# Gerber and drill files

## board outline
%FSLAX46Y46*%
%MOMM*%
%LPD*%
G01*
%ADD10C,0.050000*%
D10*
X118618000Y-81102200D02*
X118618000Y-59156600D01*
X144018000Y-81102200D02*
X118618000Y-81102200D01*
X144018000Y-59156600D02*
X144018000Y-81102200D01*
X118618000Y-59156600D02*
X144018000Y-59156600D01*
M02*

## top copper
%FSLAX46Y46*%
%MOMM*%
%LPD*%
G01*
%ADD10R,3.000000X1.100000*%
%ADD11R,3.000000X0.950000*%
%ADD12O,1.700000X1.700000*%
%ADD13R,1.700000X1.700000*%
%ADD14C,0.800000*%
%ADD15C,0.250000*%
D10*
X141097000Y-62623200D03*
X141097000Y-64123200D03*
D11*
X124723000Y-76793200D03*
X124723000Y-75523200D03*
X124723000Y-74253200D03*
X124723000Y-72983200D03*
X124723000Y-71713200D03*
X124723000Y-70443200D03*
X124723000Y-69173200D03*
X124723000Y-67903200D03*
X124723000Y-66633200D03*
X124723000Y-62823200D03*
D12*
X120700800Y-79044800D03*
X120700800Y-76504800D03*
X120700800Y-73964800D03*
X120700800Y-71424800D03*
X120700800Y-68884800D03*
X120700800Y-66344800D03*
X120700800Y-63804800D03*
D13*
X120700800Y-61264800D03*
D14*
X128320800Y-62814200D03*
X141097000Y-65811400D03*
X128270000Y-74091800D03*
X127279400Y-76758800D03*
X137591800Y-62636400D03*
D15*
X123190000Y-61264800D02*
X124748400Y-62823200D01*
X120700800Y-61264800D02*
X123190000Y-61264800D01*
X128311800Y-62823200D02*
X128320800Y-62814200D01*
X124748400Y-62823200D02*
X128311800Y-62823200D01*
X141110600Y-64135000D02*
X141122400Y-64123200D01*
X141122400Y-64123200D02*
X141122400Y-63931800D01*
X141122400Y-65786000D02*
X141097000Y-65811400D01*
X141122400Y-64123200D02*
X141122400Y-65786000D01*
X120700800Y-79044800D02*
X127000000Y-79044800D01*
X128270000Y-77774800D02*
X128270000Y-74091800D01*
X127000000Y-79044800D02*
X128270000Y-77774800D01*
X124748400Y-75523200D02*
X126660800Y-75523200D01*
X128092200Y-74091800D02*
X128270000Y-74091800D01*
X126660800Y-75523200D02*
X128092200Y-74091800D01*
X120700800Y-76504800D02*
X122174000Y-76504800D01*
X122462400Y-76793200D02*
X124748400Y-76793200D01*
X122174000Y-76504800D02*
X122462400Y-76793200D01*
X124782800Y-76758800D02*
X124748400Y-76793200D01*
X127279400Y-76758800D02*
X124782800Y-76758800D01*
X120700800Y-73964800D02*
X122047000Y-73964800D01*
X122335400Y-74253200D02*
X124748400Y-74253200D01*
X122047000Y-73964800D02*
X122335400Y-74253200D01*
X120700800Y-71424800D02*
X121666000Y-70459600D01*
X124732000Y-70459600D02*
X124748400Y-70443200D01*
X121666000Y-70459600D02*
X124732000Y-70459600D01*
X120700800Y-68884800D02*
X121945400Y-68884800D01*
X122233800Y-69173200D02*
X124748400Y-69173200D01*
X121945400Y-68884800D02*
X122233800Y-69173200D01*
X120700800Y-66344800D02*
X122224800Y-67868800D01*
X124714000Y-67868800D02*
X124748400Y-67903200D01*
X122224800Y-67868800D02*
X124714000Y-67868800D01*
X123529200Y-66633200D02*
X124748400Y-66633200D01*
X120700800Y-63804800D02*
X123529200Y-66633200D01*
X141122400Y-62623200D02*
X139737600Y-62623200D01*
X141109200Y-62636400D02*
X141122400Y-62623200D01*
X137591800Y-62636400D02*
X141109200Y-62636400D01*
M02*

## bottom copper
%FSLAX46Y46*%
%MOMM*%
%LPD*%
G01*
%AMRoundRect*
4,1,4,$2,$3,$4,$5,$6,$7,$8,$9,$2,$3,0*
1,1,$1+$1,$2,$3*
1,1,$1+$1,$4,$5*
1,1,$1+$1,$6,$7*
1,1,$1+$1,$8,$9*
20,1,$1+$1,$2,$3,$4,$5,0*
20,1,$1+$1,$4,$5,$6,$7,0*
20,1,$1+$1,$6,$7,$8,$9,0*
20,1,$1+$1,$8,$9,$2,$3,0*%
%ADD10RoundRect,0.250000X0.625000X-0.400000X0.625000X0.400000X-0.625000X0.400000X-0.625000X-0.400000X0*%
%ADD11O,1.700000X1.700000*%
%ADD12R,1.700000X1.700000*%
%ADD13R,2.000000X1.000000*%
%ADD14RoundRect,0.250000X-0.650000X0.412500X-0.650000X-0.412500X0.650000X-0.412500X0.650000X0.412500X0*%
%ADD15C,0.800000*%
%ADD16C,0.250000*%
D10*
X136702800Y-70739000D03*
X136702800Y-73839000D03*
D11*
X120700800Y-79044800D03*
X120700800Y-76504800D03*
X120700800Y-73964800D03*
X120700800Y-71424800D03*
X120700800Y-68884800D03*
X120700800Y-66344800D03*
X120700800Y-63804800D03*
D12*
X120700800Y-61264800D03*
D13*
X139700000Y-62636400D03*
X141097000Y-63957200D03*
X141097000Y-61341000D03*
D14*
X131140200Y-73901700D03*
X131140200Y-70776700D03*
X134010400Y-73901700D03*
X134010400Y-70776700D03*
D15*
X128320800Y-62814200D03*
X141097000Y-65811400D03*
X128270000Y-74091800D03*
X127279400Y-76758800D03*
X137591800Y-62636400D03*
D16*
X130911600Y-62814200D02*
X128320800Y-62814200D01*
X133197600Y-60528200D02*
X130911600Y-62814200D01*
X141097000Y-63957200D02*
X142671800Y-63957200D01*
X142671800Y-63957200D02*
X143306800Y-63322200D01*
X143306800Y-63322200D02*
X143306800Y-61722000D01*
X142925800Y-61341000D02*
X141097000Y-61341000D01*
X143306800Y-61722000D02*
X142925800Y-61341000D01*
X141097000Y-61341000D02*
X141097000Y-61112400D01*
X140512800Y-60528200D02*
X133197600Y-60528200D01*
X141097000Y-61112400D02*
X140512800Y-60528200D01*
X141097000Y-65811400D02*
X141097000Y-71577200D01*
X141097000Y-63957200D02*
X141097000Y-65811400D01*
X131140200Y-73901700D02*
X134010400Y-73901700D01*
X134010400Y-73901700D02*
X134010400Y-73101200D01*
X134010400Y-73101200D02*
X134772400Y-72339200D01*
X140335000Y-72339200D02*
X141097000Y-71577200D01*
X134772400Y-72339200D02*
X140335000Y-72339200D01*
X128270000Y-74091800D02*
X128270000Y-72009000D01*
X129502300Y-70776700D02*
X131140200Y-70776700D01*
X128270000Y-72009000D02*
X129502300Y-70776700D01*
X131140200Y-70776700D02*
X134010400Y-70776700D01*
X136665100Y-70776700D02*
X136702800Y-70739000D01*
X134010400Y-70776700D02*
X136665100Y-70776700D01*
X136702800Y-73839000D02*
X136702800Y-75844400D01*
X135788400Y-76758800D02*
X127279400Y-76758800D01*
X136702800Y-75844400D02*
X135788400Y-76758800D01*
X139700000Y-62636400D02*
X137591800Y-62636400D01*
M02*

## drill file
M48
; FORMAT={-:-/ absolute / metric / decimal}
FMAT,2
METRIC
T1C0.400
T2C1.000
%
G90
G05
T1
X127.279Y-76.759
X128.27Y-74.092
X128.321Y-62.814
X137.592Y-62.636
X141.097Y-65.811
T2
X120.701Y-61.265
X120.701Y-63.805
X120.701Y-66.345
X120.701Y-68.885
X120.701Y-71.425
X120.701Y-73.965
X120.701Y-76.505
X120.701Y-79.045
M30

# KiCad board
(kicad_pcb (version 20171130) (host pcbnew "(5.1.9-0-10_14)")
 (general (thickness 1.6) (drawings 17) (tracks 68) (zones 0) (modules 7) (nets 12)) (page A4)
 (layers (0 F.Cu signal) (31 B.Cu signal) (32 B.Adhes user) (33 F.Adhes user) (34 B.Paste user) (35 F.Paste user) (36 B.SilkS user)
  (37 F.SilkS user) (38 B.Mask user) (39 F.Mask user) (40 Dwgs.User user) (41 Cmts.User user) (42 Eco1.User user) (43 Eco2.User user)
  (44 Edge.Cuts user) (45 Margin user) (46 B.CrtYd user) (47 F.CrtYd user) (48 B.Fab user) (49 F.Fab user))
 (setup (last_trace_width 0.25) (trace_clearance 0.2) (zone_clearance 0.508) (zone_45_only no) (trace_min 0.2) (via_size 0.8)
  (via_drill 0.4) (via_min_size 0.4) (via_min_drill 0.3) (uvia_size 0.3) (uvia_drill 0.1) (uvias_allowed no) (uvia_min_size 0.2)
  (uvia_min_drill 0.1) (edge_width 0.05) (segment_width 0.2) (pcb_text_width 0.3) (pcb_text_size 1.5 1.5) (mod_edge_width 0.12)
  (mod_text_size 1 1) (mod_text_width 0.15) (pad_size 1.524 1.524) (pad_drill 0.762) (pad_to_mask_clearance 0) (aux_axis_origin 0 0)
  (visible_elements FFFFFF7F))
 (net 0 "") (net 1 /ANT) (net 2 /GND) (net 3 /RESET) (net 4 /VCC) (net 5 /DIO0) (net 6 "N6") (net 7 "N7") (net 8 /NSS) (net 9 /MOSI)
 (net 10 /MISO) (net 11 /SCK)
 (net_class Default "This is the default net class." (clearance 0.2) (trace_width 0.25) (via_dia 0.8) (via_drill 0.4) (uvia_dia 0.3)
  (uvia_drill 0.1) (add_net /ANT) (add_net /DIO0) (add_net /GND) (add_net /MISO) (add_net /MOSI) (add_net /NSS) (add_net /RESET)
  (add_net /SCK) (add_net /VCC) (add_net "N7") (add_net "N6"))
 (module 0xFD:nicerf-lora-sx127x (layer F.Cu) (at 133.223 71.3232)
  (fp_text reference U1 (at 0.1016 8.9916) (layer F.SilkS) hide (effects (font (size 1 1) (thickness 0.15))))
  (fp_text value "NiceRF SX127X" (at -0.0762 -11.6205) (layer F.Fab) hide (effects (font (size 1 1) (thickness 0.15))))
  (pad 13 smd rect (at 7.874 -8.7) (size 3 1.1) (layers F.Cu F.Paste F.Mask) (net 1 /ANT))
  (pad 14 smd rect (at 7.874 -7.2) (size 3 1.1) (layers F.Cu F.Paste F.Mask) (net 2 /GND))
  (pad 12 smd rect (at -8.5 5.47) (size 3 0.95) (layers F.Cu F.Paste F.Mask) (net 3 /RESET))
  (pad 11 smd rect (at -8.5 4.2) (size 3 0.95) (layers F.Cu F.Paste F.Mask) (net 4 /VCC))
  (pad 10 smd rect (at -8.5 2.93) (size 3 0.95) (layers F.Cu F.Paste F.Mask) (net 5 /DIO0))
  (pad 9 smd rect (at -8.5 1.66) (size 3 0.95) (layers F.Cu F.Paste F.Mask) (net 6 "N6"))
  (pad 8 smd rect (at -8.5 0.39) (size 3 0.95) (layers F.Cu F.Paste F.Mask) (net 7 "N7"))
  (pad 7 smd rect (at -8.5 -0.88) (size 3 0.95) (layers F.Cu F.Paste F.Mask) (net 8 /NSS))
  (pad 6 smd rect (at -8.5 -2.15) (size 3 0.95) (layers F.Cu F.Paste F.Mask) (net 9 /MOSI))
  (pad 5 smd rect (at -8.5 -3.42) (size 3 0.95) (layers F.Cu F.Paste F.Mask) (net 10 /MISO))
  (pad 4 smd rect (at -8.5 -4.69) (size 3 0.95) (layers F.Cu F.Paste F.Mask) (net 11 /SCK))
  (pad 1 smd rect (at -8.5 -8.5) (size 3 0.95) (layers F.Cu F.Paste F.Mask) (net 2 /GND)))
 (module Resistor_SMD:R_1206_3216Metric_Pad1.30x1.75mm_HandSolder (layer B.Cu) (at 136.7028 72.289 90)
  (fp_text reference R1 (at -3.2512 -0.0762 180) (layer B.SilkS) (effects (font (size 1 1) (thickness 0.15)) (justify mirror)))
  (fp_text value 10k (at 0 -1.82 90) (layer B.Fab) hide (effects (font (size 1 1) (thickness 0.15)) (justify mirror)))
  (pad 2 smd roundrect (at 1.55 0 90) (size 1.3 1.75) (layers B.Cu B.Paste B.Mask) (roundrect_rratio 0.192308) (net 4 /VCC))
  (pad 1 smd roundrect (at -1.55 0 90) (size 1.3 1.75) (layers B.Cu B.Paste B.Mask) (roundrect_rratio 0.192308) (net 3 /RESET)))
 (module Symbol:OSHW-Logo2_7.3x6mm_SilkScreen (layer B.Cu) (at 132.9944 64.2366 180)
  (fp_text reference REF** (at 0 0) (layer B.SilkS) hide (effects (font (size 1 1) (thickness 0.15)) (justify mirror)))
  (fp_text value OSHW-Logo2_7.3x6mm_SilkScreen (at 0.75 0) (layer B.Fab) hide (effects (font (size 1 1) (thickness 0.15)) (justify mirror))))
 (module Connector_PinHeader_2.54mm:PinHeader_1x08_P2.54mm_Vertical (layer F.Cu) (at 120.7008 61.2648)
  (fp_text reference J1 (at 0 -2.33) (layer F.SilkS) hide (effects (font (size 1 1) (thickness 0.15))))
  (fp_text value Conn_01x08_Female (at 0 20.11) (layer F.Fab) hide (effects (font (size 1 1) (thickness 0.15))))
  (pad 8 thru_hole oval (at 0 17.78) (size 1.7 1.7) (drill 1) (layers *.Cu *.Mask) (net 4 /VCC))
  (pad 7 thru_hole oval (at 0 15.24) (size 1.7 1.7) (drill 1) (layers *.Cu *.Mask) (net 3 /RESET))
  (pad 6 thru_hole oval (at 0 12.7) (size 1.7 1.7) (drill 1) (layers *.Cu *.Mask) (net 5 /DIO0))
  (pad 5 thru_hole oval (at 0 10.16) (size 1.7 1.7) (drill 1) (layers *.Cu *.Mask) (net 8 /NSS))
  (pad 4 thru_hole oval (at 0 7.62) (size 1.7 1.7) (drill 1) (layers *.Cu *.Mask) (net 9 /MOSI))
  (pad 3 thru_hole oval (at 0 5.08) (size 1.7 1.7) (drill 1) (layers *.Cu *.Mask) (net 10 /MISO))
  (pad 2 thru_hole oval (at 0 2.54) (size 1.7 1.7) (drill 1) (layers *.Cu *.Mask) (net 11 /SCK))
  (pad 1 thru_hole rect (at 0 0) (size 1.7 1.7) (drill 1) (layers *.Cu *.Mask) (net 2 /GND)))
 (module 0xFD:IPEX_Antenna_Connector (layer B.Cu) (at 141.097 62.6618 270)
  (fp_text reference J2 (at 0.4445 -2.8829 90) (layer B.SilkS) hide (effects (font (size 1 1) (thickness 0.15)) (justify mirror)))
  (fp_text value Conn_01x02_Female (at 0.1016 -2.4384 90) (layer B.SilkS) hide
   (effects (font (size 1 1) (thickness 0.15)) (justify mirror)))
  (pad 2 smd rect (at -0.0254 1.397) (size 2 1) (layers B.Cu B.Paste B.Mask) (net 1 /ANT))
  (pad 1 smd rect (at 1.2954 0 270) (size 1 2) (layers B.Cu B.Paste B.Mask) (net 2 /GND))
  (pad 1 smd rect (at -1.3208 0) (size 2 1) (layers B.Cu B.Paste B.Mask) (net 2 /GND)))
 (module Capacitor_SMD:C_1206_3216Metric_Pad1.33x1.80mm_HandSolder (layer B.Cu) (at 131.1402 72.3392 270)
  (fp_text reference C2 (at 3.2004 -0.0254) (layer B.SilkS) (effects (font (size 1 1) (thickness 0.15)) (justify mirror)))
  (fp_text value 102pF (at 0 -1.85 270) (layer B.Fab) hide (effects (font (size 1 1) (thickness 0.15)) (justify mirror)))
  (pad 2 smd roundrect (at 1.5625 0 270) (size 1.325 1.8) (layers B.Cu B.Paste B.Mask) (roundrect_rratio 0.188679) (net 2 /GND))
  (pad 1 smd roundrect (at -1.5625 0 270) (size 1.325 1.8) (layers B.Cu B.Paste B.Mask) (roundrect_rratio 0.188679) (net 4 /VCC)))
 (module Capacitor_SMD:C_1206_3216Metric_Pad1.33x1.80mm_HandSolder (layer B.Cu) (at 134.0104 72.3392 270)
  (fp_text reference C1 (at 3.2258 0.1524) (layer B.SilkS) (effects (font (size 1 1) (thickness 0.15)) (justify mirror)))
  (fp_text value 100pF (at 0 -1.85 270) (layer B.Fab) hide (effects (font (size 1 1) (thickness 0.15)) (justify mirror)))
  (pad 2 smd roundrect (at 1.5625 0 270) (size 1.325 1.8) (layers B.Cu B.Paste B.Mask) (roundrect_rratio 0.188679) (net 2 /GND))
  (pad 1 smd roundrect (at -1.5625 0 270) (size 1.325 1.8) (layers B.Cu B.Paste B.Mask) (roundrect_rratio 0.188679) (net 4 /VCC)))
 (gr_line (start 118.618 81.1022) (end 118.618 59.1566) (layer Edge.Cuts) (width 0.05))
 (gr_line (start 144.018 81.1022) (end 118.618 81.1022) (layer Edge.Cuts) (width 0.05))
 (gr_line (start 144.018 59.1566) (end 144.018 81.1022) (layer Edge.Cuts) (width 0.05))
 (gr_line (start 118.618 59.1566) (end 144.018 59.1566) (layer Edge.Cuts) (width 0.05))
 (segment (start 123.19 61.2648) (end 124.7484 62.8232) (width 0.25) (layer F.Cu) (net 2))
 (segment (start 120.7008 61.2648) (end 123.19 61.2648) (width 0.25) (layer F.Cu) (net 2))
 (via (at 128.3208 62.8142) (size 0.8) (drill 0.4) (layers F.Cu B.Cu) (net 2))
 (segment (start 128.3118 62.8232) (end 128.3208 62.8142) (width 0.25) (layer F.Cu) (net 2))
 (segment (start 124.7484 62.8232) (end 128.3118 62.8232) (width 0.25) (layer F.Cu) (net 2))
 (segment (start 130.9116 62.8142) (end 128.3208 62.8142) (width 0.25) (layer B.Cu) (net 2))
 (segment (start 141.1106 64.135) (end 141.1224 64.1232) (width 0.25) (layer F.Cu) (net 2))
 (segment (start 141.1224 64.1232) (end 141.1224 63.9318) (width 0.25) (layer F.Cu) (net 2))
 (segment (start 133.1976 60.5282) (end 130.9116 62.8142) (width 0.25) (layer B.Cu) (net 2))
 (segment (start 141.097 63.9572) (end 142.6718 63.9572) (width 0.25) (layer B.Cu) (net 2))
 (segment (start 142.6718 63.9572) (end 143.3068 63.3222) (width 0.25) (layer B.Cu) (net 2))
 (segment (start 143.3068 63.3222) (end 143.3068 61.722) (width 0.25) (layer B.Cu) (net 2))
 (segment (start 142.9258 61.341) (end 141.097 61.341) (width 0.25) (layer B.Cu) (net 2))
 (segment (start 143.3068 61.722) (end 142.9258 61.341) (width 0.25) (layer B.Cu) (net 2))
 (segment (start 141.097 61.341) (end 141.097 61.1124) (width 0.25) (layer B.Cu) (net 2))
 (segment (start 140.5128 60.5282) (end 133.1976 60.5282) (width 0.25) (layer B.Cu) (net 2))
 (segment (start 141.097 61.1124) (end 140.5128 60.5282) (width 0.25) (layer B.Cu) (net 2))
 (segment (start 141.1224 65.786) (end 141.097 65.8114) (width 0.25) (layer F.Cu) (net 2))
 (via (at 141.097 65.8114) (size 0.8) (drill 0.4) (layers F.Cu B.Cu) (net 2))
 (segment (start 141.1224 64.1232) (end 141.1224 65.786) (width 0.25) (layer F.Cu) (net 2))
 (segment (start 141.097 65.8114) (end 141.097 71.5772) (width 0.25) (layer B.Cu) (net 2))
 (segment (start 141.097 63.9572) (end 141.097 65.8114) (width 0.25) (layer B.Cu) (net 2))
 (segment (start 131.1402 73.9017) (end 134.0104 73.9017) (width 0.25) (layer B.Cu) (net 2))
 (segment (start 134.0104 73.9017) (end 134.0104 73.1012) (width 0.25) (layer B.Cu) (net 2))
 (segment (start 134.0104 73.1012) (end 134.7724 72.3392) (width 0.25) (layer B.Cu) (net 2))
 (segment (start 140.335 72.3392) (end 141.097 71.5772) (width 0.25) (layer B.Cu) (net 2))
 (segment (start 134.7724 72.3392) (end 140.335 72.3392) (width 0.25) (layer B.Cu) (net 2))
 (via (at 128.27 74.0918) (size 0.8) (drill 0.4) (layers F.Cu B.Cu) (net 4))
 (segment (start 120.7008 79.0448) (end 127 79.0448) (width 0.25) (layer F.Cu) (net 4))
 (segment (start 128.27 77.7748) (end 128.27 74.0918) (width 0.25) (layer F.Cu) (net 4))
 (segment (start 127 79.0448) (end 128.27 77.7748) (width 0.25) (layer F.Cu) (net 4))
 (segment (start 124.7484 75.5232) (end 126.6608 75.5232) (width 0.25) (layer F.Cu) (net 4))
 (segment (start 128.0922 74.0918) (end 128.27 74.0918) (width 0.25) (layer F.Cu) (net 4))
 (segment (start 126.6608 75.5232) (end 128.0922 74.0918) (width 0.25) (layer F.Cu) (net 4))
 (segment (start 128.27 74.0918) (end 128.27 72.009) (width 0.25) (layer B.Cu) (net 4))
 (segment (start 129.5023 70.7767) (end 131.1402 70.7767) (width 0.25) (layer B.Cu) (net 4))
 (segment (start 128.27 72.009) (end 129.5023 70.7767) (width 0.25) (layer B.Cu) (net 4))
 (segment (start 131.1402 70.7767) (end 134.0104 70.7767) (width 0.25) (layer B.Cu) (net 4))
 (segment (start 136.6651 70.7767) (end 136.7028 70.739) (width 0.25) (layer B.Cu) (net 4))
 (segment (start 134.0104 70.7767) (end 136.6651 70.7767) (width 0.25) (layer B.Cu) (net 4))
 (segment (start 120.7008 76.5048) (end 122.174 76.5048) (width 0.25) (layer F.Cu) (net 3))
 (segment (start 122.4624 76.7932) (end 124.7484 76.7932) (width 0.25) (layer F.Cu) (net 3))
 (segment (start 122.174 76.5048) (end 122.4624 76.7932) (width 0.25) (layer F.Cu) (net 3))
 (via (at 127.2794 76.7588) (size 0.8) (drill 0.4) (layers F.Cu B.Cu) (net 3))
 (segment (start 124.7828 76.7588) (end 124.7484 76.7932) (width 0.25) (layer F.Cu) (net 3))
 (segment (start 127.2794 76.7588) (end 124.7828 76.7588) (width 0.25) (layer F.Cu) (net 3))
 (segment (start 136.7028 73.839) (end 136.7028 75.8444) (width 0.25) (layer B.Cu) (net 3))
 (segment (start 135.7884 76.7588) (end 127.2794 76.7588) (width 0.25) (layer B.Cu) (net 3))
 (segment (start 136.7028 75.8444) (end 135.7884 76.7588) (width 0.25) (layer B.Cu) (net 3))
 (segment (start 120.7008 73.9648) (end 122.047 73.9648) (width 0.25) (layer F.Cu) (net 5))
 (segment (start 122.3354 74.2532) (end 124.7484 74.2532) (width 0.25) (layer F.Cu) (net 5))
 (segment (start 122.047 73.9648) (end 122.3354 74.2532) (width 0.25) (layer F.Cu) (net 5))
 (segment (start 120.7008 71.4248) (end 121.666 70.4596) (width 0.25) (layer F.Cu) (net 8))
 (segment (start 124.732 70.4596) (end 124.7484 70.4432) (width 0.25) (layer F.Cu) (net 8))
 (segment (start 121.666 70.4596) (end 124.732 70.4596) (width 0.25) (layer F.Cu) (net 8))
 (segment (start 120.7008 68.8848) (end 121.9454 68.8848) (width 0.25) (layer F.Cu) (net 9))
 (segment (start 122.2338 69.1732) (end 124.7484 69.1732) (width 0.25) (layer F.Cu) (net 9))
 (segment (start 121.9454 68.8848) (end 122.2338 69.1732) (width 0.25) (layer F.Cu) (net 9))
 (segment (start 120.7008 66.3448) (end 122.2248 67.8688) (width 0.25) (layer F.Cu) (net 10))
 (segment (start 124.714 67.8688) (end 124.7484 67.9032) (width 0.25) (layer F.Cu) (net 10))
 (segment (start 122.2248 67.8688) (end 124.714 67.8688) (width 0.25) (layer F.Cu) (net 10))
 (segment (start 123.5292 66.6332) (end 124.7484 66.6332) (width 0.25) (layer F.Cu) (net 11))
 (segment (start 120.7008 63.8048) (end 123.5292 66.6332) (width 0.25) (layer F.Cu) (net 11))
 (segment (start 141.1224 62.6232) (end 139.7376 62.6232) (width 0.25) (layer F.Cu) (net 1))
 (via (at 137.5918 62.6364) (size 0.8) (drill 0.4) (layers F.Cu B.Cu) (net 1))
 (segment (start 139.7 62.6364) (end 137.5918 62.6364) (width 0.25) (layer B.Cu) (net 1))
 (segment (start 141.1092 62.6364) (end 141.1224 62.6232) (width 0.25) (layer F.Cu) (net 1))
 (segment (start 137.5918 62.6364) (end 141.1092 62.6364) (width 0.25) (layer F.Cu) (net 1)))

